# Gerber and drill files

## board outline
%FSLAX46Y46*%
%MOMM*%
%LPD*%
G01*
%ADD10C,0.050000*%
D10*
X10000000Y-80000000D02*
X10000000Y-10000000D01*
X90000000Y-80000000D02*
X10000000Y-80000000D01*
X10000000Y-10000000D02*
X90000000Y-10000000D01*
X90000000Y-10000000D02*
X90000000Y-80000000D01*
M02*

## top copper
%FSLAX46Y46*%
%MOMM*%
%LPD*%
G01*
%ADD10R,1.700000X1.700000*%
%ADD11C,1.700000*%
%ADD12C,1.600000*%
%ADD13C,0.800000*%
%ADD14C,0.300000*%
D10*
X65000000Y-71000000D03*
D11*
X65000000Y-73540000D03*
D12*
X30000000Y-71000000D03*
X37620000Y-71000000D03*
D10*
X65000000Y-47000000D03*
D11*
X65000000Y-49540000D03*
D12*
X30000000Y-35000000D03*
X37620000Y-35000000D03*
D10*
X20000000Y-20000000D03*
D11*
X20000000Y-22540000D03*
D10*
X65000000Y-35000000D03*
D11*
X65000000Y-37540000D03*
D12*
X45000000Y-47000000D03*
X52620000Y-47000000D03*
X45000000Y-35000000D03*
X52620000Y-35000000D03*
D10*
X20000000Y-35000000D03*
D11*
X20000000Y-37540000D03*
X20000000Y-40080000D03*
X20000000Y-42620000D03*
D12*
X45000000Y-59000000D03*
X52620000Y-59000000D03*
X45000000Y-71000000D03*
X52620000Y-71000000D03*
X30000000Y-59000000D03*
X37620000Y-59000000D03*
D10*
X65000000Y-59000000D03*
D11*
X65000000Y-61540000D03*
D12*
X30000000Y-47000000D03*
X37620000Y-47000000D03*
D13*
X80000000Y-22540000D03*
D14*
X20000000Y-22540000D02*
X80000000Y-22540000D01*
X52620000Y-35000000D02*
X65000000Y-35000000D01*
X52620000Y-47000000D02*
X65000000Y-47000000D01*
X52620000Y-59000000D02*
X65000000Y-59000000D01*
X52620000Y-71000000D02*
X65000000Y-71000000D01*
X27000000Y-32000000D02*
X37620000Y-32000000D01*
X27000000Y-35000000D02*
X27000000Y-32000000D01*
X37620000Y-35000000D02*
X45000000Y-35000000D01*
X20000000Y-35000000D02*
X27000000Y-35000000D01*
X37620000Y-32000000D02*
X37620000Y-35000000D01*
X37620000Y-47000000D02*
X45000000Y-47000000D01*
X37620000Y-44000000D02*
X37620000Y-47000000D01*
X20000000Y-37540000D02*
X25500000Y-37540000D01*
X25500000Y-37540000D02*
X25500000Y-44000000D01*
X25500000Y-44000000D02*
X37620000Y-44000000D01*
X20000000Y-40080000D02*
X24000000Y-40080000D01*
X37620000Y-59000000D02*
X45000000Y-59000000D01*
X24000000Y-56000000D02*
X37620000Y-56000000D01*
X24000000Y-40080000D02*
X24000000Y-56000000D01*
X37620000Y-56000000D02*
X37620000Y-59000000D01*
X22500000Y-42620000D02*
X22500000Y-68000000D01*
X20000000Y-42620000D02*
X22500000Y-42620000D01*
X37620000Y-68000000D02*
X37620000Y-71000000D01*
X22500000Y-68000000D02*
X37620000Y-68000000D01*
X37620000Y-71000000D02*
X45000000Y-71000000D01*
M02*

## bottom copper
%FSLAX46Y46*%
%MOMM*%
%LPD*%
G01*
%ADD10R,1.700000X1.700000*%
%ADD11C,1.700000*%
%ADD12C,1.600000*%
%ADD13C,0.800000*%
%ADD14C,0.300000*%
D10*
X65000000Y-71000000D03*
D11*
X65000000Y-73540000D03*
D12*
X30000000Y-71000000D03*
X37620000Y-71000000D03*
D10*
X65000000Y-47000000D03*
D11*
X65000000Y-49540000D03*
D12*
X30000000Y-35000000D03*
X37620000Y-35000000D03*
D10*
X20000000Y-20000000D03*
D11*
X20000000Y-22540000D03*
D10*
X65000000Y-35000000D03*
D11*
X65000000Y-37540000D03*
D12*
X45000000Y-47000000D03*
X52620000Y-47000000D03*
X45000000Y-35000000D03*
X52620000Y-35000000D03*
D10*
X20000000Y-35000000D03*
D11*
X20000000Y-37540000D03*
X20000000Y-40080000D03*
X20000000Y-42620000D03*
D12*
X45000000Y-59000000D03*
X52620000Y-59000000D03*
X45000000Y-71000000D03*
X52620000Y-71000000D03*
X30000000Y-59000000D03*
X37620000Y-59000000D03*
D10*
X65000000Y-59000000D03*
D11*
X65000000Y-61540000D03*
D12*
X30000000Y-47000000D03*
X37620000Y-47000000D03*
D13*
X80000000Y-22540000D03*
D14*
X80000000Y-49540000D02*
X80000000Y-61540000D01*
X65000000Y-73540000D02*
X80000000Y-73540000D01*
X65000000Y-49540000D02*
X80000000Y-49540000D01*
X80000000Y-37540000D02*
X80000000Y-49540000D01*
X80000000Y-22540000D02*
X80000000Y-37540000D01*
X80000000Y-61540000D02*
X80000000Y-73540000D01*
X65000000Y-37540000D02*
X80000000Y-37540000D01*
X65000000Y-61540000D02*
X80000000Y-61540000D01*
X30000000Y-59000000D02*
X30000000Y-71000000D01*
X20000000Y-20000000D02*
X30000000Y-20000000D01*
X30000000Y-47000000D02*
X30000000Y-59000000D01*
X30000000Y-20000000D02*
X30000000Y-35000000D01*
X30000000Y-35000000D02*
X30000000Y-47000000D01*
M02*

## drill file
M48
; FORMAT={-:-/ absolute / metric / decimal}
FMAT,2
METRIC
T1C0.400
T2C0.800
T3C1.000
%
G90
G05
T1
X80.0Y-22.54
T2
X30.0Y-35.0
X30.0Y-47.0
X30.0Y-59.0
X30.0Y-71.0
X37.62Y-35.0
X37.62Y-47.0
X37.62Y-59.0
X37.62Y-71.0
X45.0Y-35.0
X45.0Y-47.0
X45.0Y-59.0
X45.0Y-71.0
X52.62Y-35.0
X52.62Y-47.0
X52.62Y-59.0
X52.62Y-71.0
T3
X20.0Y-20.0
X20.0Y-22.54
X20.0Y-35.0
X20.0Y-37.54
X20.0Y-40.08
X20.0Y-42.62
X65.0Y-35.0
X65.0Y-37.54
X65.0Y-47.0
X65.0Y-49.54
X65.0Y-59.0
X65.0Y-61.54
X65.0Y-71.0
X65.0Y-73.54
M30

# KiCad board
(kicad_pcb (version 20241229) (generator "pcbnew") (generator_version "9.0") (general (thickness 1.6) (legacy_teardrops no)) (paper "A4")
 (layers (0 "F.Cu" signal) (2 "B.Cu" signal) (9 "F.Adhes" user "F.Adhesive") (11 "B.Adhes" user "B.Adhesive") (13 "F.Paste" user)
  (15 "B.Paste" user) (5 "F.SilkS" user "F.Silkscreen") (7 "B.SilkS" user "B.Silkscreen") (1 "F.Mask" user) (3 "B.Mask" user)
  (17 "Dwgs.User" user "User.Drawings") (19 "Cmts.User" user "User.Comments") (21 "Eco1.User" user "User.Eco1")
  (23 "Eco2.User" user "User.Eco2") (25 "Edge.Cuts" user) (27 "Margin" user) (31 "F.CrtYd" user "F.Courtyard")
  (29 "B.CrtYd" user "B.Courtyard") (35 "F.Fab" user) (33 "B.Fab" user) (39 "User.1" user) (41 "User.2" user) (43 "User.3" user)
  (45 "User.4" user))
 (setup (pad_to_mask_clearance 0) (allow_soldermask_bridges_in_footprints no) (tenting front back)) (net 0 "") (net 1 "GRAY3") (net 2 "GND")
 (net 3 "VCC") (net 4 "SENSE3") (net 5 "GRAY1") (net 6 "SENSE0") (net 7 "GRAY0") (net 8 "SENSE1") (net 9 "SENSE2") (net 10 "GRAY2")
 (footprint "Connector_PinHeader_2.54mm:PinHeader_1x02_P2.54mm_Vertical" (layer "F.Cu") (at 65 71)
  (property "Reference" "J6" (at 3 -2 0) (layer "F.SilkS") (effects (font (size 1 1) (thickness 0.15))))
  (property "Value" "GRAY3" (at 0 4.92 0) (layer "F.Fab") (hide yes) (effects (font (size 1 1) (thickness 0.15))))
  (pad "1" thru_hole rect (at 0 0) (size 1.7 1.7) (drill 1) (layers "*.Cu" "*.Mask") (remove_unused_layers no) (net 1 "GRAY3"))
  (pad "2" thru_hole circle (at 0 2.54) (size 1.7 1.7) (drill 1) (layers "*.Cu" "*.Mask") (remove_unused_layers no) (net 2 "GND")))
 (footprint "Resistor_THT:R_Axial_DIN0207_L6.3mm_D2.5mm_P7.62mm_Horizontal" (layer "F.Cu") (at 30 71)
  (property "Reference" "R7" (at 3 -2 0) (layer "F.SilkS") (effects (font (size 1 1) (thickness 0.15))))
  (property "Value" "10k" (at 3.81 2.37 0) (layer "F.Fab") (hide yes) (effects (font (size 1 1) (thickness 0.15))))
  (pad "1" thru_hole circle (at 0 0) (size 1.6 1.6) (drill 0.8) (layers "*.Cu" "*.Mask") (remove_unused_layers no) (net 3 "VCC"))
  (pad "2" thru_hole circle (at 7.62 0) (size 1.6 1.6) (drill 0.8) (layers "*.Cu" "*.Mask") (remove_unused_layers no) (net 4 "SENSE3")))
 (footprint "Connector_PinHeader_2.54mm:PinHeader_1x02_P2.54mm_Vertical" (layer "F.Cu") (at 65 47)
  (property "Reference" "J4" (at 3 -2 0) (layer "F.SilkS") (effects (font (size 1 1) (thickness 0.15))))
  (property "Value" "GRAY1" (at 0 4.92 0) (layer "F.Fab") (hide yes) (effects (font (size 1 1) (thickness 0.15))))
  (pad "1" thru_hole rect (at 0 0) (size 1.7 1.7) (drill 1) (layers "*.Cu" "*.Mask") (remove_unused_layers no) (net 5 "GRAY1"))
  (pad "2" thru_hole circle (at 0 2.54) (size 1.7 1.7) (drill 1) (layers "*.Cu" "*.Mask") (remove_unused_layers no) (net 2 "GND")))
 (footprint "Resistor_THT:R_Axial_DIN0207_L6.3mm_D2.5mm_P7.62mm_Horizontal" (layer "F.Cu") (at 30 35)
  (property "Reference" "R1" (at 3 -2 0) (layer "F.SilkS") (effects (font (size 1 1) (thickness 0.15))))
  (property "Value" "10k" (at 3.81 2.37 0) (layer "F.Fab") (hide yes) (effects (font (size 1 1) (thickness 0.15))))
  (pad "1" thru_hole circle (at 0 0) (size 1.6 1.6) (drill 0.8) (layers "*.Cu" "*.Mask") (remove_unused_layers no) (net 3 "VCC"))
  (pad "2" thru_hole circle (at 7.62 0) (size 1.6 1.6) (drill 0.8) (layers "*.Cu" "*.Mask") (remove_unused_layers no) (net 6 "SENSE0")))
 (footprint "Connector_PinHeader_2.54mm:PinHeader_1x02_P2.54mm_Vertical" (layer "F.Cu") (at 20 20)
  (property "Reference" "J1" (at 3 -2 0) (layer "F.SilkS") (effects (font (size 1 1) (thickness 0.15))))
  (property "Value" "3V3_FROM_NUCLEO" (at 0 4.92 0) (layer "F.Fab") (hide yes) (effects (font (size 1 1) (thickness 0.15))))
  (pad "1" thru_hole rect (at 0 0) (size 1.7 1.7) (drill 1) (layers "*.Cu" "*.Mask") (remove_unused_layers no) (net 3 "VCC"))
  (pad "2" thru_hole circle (at 0 2.54) (size 1.7 1.7) (drill 1) (layers "*.Cu" "*.Mask") (remove_unused_layers no) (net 2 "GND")))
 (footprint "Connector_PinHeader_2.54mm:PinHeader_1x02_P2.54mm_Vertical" (layer "F.Cu") (at 65 35)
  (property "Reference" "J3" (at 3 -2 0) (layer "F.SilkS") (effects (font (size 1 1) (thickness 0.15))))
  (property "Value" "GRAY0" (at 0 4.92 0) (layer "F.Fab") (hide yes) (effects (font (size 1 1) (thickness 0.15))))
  (pad "1" thru_hole rect (at 0 0) (size 1.7 1.7) (drill 1) (layers "*.Cu" "*.Mask") (remove_unused_layers no) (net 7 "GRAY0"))
  (pad "2" thru_hole circle (at 0 2.54) (size 1.7 1.7) (drill 1) (layers "*.Cu" "*.Mask") (remove_unused_layers no) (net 2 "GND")))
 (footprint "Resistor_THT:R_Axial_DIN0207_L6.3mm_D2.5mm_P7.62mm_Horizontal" (layer "F.Cu") (at 45 47)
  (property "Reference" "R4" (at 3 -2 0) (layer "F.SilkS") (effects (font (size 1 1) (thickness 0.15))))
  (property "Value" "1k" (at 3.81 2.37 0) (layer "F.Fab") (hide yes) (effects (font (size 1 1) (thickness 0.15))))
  (pad "1" thru_hole circle (at 0 0) (size 1.6 1.6) (drill 0.8) (layers "*.Cu" "*.Mask") (remove_unused_layers no) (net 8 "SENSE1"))
  (pad "2" thru_hole circle (at 7.62 0) (size 1.6 1.6) (drill 0.8) (layers "*.Cu" "*.Mask") (remove_unused_layers no) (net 5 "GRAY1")))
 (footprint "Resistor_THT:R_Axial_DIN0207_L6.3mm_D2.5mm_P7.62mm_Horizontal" (layer "F.Cu") (at 45 35)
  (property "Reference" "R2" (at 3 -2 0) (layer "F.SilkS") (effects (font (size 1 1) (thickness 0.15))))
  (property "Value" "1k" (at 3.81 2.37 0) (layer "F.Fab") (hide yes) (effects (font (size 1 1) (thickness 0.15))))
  (pad "1" thru_hole circle (at 0 0) (size 1.6 1.6) (drill 0.8) (layers "*.Cu" "*.Mask") (remove_unused_layers no) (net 6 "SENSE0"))
  (pad "2" thru_hole circle (at 7.62 0) (size 1.6 1.6) (drill 0.8) (layers "*.Cu" "*.Mask") (remove_unused_layers no) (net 7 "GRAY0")))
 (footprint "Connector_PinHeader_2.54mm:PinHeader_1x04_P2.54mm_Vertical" (layer "F.Cu") (at 20 35)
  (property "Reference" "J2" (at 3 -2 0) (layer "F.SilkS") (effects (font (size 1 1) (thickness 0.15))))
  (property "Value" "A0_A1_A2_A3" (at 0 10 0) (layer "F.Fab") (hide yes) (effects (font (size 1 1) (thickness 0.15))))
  (pad "1" thru_hole rect (at 0 0) (size 1.7 1.7) (drill 1) (layers "*.Cu" "*.Mask") (remove_unused_layers no) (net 6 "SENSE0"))
  (pad "2" thru_hole circle (at 0 2.54) (size 1.7 1.7) (drill 1) (layers "*.Cu" "*.Mask") (remove_unused_layers no) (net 8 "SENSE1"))
  (pad "3" thru_hole circle (at 0 5.08) (size 1.7 1.7) (drill 1) (layers "*.Cu" "*.Mask") (remove_unused_layers no) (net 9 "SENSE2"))
  (pad "4" thru_hole circle (at 0 7.62) (size 1.7 1.7) (drill 1) (layers "*.Cu" "*.Mask") (remove_unused_layers no) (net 4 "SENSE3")))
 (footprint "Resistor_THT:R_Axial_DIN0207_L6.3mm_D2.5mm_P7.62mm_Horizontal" (layer "F.Cu") (at 45 59)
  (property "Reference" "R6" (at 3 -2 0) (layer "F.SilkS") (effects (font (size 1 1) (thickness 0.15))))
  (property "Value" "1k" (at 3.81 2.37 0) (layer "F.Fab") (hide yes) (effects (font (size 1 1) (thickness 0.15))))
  (pad "1" thru_hole circle (at 0 0) (size 1.6 1.6) (drill 0.8) (layers "*.Cu" "*.Mask") (remove_unused_layers no) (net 9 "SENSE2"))
  (pad "2" thru_hole circle (at 7.62 0) (size 1.6 1.6) (drill 0.8) (layers "*.Cu" "*.Mask") (remove_unused_layers no) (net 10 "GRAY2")))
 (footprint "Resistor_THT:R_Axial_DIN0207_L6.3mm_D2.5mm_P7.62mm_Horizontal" (layer "F.Cu") (at 45 71)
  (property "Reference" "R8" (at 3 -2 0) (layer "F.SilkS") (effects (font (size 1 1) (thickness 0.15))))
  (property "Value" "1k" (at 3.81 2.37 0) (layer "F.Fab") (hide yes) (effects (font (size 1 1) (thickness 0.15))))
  (pad "1" thru_hole circle (at 0 0) (size 1.6 1.6) (drill 0.8) (layers "*.Cu" "*.Mask") (remove_unused_layers no) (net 4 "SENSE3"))
  (pad "2" thru_hole circle (at 7.62 0) (size 1.6 1.6) (drill 0.8) (layers "*.Cu" "*.Mask") (remove_unused_layers no) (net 1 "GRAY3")))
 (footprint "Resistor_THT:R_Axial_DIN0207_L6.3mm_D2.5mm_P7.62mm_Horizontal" (layer "F.Cu") (at 30 59)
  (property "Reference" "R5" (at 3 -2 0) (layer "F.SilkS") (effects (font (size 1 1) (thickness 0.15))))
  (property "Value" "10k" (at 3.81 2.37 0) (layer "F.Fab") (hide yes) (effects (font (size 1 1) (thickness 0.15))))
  (pad "1" thru_hole circle (at 0 0) (size 1.6 1.6) (drill 0.8) (layers "*.Cu" "*.Mask") (remove_unused_layers no) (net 3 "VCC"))
  (pad "2" thru_hole circle (at 7.62 0) (size 1.6 1.6) (drill 0.8) (layers "*.Cu" "*.Mask") (remove_unused_layers no) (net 9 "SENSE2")))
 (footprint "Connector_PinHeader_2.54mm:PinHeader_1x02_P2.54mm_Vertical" (layer "F.Cu") (at 65 59)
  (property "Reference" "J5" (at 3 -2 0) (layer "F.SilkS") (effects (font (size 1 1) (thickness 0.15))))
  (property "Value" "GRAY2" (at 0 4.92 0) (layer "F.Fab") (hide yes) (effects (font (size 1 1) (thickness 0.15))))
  (pad "1" thru_hole rect (at 0 0) (size 1.7 1.7) (drill 1) (layers "*.Cu" "*.Mask") (remove_unused_layers no) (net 10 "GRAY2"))
  (pad "2" thru_hole circle (at 0 2.54) (size 1.7 1.7) (drill 1) (layers "*.Cu" "*.Mask") (remove_unused_layers no) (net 2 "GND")))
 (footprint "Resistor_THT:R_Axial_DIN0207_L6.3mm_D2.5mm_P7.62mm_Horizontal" (layer "F.Cu") (at 30 47)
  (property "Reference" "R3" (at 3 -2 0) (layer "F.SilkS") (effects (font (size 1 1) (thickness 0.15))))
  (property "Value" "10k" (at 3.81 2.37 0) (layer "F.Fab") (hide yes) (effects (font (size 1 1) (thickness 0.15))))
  (pad "1" thru_hole circle (at 0 0) (size 1.6 1.6) (drill 0.8) (layers "*.Cu" "*.Mask") (remove_unused_layers no) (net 3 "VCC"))
  (pad "2" thru_hole circle (at 7.62 0) (size 1.6 1.6) (drill 0.8) (layers "*.Cu" "*.Mask") (remove_unused_layers no) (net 8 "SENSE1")))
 (gr_line (start 10 80) (end 10 10) (stroke (width 0.05) (type default)) (layer "Edge.Cuts"))
 (gr_line (start 90 80) (end 10 80) (stroke (width 0.05) (type default)) (layer "Edge.Cuts"))
 (gr_line (start 10 10) (end 90 10) (stroke (width 0.05) (type default)) (layer "Edge.Cuts"))
 (gr_line (start 90 10) (end 90 80) (stroke (width 0.05) (type default)) (layer "Edge.Cuts"))
 (segment (start 20 22.54) (end 80 22.54) (width 0.3) (layer "F.Cu") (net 2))
 (via (at 80 22.54) (size 0.8) (drill 0.4) (layers "F.Cu" "B.Cu") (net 2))
 (segment (start 80 49.54) (end 80 61.54) (width 0.3) (layer "B.Cu") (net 2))
 (segment (start 65 73.54) (end 80 73.54) (width 0.3) (layer "B.Cu") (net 2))
 (segment (start 65 49.54) (end 80 49.54) (width 0.3) (layer "B.Cu") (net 2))
 (segment (start 80 37.54) (end 80 49.54) (width 0.3) (layer "B.Cu") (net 2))
 (segment (start 80 22.54) (end 80 37.54) (width 0.3) (layer "B.Cu") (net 2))
 (segment (start 80 61.54) (end 80 73.54) (width 0.3) (layer "B.Cu") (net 2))
 (segment (start 65 37.54) (end 80 37.54) (width 0.3) (layer "B.Cu") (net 2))
 (segment (start 65 61.54) (end 80 61.54) (width 0.3) (layer "B.Cu") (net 2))
 (segment (start 52.62 35) (end 65 35) (width 0.3) (layer "F.Cu") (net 7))
 (segment (start 52.62 47) (end 65 47) (width 0.3) (layer "F.Cu") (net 5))
 (segment (start 52.62 59) (end 65 59) (width 0.3) (layer "F.Cu") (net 10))
 (segment (start 52.62 71) (end 65 71) (width 0.3) (layer "F.Cu") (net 1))
 (segment (start 27 32) (end 37.62 32) (width 0.3) (layer "F.Cu") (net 6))
 (segment (start 27 35) (end 27 32) (width 0.3) (layer "F.Cu") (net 6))
 (segment (start 37.62 35) (end 45 35) (width 0.3) (layer "F.Cu") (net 6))
 (segment (start 20 35) (end 27 35) (width 0.3) (layer "F.Cu") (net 6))
 (segment (start 37.62 32) (end 37.62 35) (width 0.3) (layer "F.Cu") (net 6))
 (segment (start 37.62 47) (end 45 47) (width 0.3) (layer "F.Cu") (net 8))
 (segment (start 37.62 44) (end 37.62 47) (width 0.3) (layer "F.Cu") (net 8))
 (segment (start 20 37.54) (end 25.5 37.54) (width 0.3) (layer "F.Cu") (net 8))
 (segment (start 25.5 37.54) (end 25.5 44) (width 0.3) (layer "F.Cu") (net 8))
 (segment (start 25.5 44) (end 37.62 44) (width 0.3) (layer "F.Cu") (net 8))
 (segment (start 20 40.08) (end 24 40.08) (width 0.3) (layer "F.Cu") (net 9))
 (segment (start 37.62 59) (end 45 59) (width 0.3) (layer "F.Cu") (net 9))
 (segment (start 24 56) (end 37.62 56) (width 0.3) (layer "F.Cu") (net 9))
 (segment (start 24 40.08) (end 24 56) (width 0.3) (layer "F.Cu") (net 9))
 (segment (start 37.62 56) (end 37.62 59) (width 0.3) (layer "F.Cu") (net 9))
 (segment (start 22.5 42.62) (end 22.5 68) (width 0.3) (layer "F.Cu") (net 4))
 (segment (start 20 42.62) (end 22.5 42.62) (width 0.3) (layer "F.Cu") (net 4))
 (segment (start 37.62 68) (end 37.62 71) (width 0.3) (layer "F.Cu") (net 4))
 (segment (start 22.5 68) (end 37.62 68) (width 0.3) (layer "F.Cu") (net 4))
 (segment (start 37.62 71) (end 45 71) (width 0.3) (layer "F.Cu") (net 4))
 (segment (start 30 59) (end 30 71) (width 0.3) (layer "B.Cu") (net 3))
 (segment (start 20 20) (end 30 20) (width 0.3) (layer "B.Cu") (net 3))
 (segment (start 30 47) (end 30 59) (width 0.3) (layer "B.Cu") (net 3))
 (segment (start 30 20) (end 30 35) (width 0.3) (layer "B.Cu") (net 3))
 (segment (start 30 35) (end 30 47) (width 0.3) (layer "B.Cu") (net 3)))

